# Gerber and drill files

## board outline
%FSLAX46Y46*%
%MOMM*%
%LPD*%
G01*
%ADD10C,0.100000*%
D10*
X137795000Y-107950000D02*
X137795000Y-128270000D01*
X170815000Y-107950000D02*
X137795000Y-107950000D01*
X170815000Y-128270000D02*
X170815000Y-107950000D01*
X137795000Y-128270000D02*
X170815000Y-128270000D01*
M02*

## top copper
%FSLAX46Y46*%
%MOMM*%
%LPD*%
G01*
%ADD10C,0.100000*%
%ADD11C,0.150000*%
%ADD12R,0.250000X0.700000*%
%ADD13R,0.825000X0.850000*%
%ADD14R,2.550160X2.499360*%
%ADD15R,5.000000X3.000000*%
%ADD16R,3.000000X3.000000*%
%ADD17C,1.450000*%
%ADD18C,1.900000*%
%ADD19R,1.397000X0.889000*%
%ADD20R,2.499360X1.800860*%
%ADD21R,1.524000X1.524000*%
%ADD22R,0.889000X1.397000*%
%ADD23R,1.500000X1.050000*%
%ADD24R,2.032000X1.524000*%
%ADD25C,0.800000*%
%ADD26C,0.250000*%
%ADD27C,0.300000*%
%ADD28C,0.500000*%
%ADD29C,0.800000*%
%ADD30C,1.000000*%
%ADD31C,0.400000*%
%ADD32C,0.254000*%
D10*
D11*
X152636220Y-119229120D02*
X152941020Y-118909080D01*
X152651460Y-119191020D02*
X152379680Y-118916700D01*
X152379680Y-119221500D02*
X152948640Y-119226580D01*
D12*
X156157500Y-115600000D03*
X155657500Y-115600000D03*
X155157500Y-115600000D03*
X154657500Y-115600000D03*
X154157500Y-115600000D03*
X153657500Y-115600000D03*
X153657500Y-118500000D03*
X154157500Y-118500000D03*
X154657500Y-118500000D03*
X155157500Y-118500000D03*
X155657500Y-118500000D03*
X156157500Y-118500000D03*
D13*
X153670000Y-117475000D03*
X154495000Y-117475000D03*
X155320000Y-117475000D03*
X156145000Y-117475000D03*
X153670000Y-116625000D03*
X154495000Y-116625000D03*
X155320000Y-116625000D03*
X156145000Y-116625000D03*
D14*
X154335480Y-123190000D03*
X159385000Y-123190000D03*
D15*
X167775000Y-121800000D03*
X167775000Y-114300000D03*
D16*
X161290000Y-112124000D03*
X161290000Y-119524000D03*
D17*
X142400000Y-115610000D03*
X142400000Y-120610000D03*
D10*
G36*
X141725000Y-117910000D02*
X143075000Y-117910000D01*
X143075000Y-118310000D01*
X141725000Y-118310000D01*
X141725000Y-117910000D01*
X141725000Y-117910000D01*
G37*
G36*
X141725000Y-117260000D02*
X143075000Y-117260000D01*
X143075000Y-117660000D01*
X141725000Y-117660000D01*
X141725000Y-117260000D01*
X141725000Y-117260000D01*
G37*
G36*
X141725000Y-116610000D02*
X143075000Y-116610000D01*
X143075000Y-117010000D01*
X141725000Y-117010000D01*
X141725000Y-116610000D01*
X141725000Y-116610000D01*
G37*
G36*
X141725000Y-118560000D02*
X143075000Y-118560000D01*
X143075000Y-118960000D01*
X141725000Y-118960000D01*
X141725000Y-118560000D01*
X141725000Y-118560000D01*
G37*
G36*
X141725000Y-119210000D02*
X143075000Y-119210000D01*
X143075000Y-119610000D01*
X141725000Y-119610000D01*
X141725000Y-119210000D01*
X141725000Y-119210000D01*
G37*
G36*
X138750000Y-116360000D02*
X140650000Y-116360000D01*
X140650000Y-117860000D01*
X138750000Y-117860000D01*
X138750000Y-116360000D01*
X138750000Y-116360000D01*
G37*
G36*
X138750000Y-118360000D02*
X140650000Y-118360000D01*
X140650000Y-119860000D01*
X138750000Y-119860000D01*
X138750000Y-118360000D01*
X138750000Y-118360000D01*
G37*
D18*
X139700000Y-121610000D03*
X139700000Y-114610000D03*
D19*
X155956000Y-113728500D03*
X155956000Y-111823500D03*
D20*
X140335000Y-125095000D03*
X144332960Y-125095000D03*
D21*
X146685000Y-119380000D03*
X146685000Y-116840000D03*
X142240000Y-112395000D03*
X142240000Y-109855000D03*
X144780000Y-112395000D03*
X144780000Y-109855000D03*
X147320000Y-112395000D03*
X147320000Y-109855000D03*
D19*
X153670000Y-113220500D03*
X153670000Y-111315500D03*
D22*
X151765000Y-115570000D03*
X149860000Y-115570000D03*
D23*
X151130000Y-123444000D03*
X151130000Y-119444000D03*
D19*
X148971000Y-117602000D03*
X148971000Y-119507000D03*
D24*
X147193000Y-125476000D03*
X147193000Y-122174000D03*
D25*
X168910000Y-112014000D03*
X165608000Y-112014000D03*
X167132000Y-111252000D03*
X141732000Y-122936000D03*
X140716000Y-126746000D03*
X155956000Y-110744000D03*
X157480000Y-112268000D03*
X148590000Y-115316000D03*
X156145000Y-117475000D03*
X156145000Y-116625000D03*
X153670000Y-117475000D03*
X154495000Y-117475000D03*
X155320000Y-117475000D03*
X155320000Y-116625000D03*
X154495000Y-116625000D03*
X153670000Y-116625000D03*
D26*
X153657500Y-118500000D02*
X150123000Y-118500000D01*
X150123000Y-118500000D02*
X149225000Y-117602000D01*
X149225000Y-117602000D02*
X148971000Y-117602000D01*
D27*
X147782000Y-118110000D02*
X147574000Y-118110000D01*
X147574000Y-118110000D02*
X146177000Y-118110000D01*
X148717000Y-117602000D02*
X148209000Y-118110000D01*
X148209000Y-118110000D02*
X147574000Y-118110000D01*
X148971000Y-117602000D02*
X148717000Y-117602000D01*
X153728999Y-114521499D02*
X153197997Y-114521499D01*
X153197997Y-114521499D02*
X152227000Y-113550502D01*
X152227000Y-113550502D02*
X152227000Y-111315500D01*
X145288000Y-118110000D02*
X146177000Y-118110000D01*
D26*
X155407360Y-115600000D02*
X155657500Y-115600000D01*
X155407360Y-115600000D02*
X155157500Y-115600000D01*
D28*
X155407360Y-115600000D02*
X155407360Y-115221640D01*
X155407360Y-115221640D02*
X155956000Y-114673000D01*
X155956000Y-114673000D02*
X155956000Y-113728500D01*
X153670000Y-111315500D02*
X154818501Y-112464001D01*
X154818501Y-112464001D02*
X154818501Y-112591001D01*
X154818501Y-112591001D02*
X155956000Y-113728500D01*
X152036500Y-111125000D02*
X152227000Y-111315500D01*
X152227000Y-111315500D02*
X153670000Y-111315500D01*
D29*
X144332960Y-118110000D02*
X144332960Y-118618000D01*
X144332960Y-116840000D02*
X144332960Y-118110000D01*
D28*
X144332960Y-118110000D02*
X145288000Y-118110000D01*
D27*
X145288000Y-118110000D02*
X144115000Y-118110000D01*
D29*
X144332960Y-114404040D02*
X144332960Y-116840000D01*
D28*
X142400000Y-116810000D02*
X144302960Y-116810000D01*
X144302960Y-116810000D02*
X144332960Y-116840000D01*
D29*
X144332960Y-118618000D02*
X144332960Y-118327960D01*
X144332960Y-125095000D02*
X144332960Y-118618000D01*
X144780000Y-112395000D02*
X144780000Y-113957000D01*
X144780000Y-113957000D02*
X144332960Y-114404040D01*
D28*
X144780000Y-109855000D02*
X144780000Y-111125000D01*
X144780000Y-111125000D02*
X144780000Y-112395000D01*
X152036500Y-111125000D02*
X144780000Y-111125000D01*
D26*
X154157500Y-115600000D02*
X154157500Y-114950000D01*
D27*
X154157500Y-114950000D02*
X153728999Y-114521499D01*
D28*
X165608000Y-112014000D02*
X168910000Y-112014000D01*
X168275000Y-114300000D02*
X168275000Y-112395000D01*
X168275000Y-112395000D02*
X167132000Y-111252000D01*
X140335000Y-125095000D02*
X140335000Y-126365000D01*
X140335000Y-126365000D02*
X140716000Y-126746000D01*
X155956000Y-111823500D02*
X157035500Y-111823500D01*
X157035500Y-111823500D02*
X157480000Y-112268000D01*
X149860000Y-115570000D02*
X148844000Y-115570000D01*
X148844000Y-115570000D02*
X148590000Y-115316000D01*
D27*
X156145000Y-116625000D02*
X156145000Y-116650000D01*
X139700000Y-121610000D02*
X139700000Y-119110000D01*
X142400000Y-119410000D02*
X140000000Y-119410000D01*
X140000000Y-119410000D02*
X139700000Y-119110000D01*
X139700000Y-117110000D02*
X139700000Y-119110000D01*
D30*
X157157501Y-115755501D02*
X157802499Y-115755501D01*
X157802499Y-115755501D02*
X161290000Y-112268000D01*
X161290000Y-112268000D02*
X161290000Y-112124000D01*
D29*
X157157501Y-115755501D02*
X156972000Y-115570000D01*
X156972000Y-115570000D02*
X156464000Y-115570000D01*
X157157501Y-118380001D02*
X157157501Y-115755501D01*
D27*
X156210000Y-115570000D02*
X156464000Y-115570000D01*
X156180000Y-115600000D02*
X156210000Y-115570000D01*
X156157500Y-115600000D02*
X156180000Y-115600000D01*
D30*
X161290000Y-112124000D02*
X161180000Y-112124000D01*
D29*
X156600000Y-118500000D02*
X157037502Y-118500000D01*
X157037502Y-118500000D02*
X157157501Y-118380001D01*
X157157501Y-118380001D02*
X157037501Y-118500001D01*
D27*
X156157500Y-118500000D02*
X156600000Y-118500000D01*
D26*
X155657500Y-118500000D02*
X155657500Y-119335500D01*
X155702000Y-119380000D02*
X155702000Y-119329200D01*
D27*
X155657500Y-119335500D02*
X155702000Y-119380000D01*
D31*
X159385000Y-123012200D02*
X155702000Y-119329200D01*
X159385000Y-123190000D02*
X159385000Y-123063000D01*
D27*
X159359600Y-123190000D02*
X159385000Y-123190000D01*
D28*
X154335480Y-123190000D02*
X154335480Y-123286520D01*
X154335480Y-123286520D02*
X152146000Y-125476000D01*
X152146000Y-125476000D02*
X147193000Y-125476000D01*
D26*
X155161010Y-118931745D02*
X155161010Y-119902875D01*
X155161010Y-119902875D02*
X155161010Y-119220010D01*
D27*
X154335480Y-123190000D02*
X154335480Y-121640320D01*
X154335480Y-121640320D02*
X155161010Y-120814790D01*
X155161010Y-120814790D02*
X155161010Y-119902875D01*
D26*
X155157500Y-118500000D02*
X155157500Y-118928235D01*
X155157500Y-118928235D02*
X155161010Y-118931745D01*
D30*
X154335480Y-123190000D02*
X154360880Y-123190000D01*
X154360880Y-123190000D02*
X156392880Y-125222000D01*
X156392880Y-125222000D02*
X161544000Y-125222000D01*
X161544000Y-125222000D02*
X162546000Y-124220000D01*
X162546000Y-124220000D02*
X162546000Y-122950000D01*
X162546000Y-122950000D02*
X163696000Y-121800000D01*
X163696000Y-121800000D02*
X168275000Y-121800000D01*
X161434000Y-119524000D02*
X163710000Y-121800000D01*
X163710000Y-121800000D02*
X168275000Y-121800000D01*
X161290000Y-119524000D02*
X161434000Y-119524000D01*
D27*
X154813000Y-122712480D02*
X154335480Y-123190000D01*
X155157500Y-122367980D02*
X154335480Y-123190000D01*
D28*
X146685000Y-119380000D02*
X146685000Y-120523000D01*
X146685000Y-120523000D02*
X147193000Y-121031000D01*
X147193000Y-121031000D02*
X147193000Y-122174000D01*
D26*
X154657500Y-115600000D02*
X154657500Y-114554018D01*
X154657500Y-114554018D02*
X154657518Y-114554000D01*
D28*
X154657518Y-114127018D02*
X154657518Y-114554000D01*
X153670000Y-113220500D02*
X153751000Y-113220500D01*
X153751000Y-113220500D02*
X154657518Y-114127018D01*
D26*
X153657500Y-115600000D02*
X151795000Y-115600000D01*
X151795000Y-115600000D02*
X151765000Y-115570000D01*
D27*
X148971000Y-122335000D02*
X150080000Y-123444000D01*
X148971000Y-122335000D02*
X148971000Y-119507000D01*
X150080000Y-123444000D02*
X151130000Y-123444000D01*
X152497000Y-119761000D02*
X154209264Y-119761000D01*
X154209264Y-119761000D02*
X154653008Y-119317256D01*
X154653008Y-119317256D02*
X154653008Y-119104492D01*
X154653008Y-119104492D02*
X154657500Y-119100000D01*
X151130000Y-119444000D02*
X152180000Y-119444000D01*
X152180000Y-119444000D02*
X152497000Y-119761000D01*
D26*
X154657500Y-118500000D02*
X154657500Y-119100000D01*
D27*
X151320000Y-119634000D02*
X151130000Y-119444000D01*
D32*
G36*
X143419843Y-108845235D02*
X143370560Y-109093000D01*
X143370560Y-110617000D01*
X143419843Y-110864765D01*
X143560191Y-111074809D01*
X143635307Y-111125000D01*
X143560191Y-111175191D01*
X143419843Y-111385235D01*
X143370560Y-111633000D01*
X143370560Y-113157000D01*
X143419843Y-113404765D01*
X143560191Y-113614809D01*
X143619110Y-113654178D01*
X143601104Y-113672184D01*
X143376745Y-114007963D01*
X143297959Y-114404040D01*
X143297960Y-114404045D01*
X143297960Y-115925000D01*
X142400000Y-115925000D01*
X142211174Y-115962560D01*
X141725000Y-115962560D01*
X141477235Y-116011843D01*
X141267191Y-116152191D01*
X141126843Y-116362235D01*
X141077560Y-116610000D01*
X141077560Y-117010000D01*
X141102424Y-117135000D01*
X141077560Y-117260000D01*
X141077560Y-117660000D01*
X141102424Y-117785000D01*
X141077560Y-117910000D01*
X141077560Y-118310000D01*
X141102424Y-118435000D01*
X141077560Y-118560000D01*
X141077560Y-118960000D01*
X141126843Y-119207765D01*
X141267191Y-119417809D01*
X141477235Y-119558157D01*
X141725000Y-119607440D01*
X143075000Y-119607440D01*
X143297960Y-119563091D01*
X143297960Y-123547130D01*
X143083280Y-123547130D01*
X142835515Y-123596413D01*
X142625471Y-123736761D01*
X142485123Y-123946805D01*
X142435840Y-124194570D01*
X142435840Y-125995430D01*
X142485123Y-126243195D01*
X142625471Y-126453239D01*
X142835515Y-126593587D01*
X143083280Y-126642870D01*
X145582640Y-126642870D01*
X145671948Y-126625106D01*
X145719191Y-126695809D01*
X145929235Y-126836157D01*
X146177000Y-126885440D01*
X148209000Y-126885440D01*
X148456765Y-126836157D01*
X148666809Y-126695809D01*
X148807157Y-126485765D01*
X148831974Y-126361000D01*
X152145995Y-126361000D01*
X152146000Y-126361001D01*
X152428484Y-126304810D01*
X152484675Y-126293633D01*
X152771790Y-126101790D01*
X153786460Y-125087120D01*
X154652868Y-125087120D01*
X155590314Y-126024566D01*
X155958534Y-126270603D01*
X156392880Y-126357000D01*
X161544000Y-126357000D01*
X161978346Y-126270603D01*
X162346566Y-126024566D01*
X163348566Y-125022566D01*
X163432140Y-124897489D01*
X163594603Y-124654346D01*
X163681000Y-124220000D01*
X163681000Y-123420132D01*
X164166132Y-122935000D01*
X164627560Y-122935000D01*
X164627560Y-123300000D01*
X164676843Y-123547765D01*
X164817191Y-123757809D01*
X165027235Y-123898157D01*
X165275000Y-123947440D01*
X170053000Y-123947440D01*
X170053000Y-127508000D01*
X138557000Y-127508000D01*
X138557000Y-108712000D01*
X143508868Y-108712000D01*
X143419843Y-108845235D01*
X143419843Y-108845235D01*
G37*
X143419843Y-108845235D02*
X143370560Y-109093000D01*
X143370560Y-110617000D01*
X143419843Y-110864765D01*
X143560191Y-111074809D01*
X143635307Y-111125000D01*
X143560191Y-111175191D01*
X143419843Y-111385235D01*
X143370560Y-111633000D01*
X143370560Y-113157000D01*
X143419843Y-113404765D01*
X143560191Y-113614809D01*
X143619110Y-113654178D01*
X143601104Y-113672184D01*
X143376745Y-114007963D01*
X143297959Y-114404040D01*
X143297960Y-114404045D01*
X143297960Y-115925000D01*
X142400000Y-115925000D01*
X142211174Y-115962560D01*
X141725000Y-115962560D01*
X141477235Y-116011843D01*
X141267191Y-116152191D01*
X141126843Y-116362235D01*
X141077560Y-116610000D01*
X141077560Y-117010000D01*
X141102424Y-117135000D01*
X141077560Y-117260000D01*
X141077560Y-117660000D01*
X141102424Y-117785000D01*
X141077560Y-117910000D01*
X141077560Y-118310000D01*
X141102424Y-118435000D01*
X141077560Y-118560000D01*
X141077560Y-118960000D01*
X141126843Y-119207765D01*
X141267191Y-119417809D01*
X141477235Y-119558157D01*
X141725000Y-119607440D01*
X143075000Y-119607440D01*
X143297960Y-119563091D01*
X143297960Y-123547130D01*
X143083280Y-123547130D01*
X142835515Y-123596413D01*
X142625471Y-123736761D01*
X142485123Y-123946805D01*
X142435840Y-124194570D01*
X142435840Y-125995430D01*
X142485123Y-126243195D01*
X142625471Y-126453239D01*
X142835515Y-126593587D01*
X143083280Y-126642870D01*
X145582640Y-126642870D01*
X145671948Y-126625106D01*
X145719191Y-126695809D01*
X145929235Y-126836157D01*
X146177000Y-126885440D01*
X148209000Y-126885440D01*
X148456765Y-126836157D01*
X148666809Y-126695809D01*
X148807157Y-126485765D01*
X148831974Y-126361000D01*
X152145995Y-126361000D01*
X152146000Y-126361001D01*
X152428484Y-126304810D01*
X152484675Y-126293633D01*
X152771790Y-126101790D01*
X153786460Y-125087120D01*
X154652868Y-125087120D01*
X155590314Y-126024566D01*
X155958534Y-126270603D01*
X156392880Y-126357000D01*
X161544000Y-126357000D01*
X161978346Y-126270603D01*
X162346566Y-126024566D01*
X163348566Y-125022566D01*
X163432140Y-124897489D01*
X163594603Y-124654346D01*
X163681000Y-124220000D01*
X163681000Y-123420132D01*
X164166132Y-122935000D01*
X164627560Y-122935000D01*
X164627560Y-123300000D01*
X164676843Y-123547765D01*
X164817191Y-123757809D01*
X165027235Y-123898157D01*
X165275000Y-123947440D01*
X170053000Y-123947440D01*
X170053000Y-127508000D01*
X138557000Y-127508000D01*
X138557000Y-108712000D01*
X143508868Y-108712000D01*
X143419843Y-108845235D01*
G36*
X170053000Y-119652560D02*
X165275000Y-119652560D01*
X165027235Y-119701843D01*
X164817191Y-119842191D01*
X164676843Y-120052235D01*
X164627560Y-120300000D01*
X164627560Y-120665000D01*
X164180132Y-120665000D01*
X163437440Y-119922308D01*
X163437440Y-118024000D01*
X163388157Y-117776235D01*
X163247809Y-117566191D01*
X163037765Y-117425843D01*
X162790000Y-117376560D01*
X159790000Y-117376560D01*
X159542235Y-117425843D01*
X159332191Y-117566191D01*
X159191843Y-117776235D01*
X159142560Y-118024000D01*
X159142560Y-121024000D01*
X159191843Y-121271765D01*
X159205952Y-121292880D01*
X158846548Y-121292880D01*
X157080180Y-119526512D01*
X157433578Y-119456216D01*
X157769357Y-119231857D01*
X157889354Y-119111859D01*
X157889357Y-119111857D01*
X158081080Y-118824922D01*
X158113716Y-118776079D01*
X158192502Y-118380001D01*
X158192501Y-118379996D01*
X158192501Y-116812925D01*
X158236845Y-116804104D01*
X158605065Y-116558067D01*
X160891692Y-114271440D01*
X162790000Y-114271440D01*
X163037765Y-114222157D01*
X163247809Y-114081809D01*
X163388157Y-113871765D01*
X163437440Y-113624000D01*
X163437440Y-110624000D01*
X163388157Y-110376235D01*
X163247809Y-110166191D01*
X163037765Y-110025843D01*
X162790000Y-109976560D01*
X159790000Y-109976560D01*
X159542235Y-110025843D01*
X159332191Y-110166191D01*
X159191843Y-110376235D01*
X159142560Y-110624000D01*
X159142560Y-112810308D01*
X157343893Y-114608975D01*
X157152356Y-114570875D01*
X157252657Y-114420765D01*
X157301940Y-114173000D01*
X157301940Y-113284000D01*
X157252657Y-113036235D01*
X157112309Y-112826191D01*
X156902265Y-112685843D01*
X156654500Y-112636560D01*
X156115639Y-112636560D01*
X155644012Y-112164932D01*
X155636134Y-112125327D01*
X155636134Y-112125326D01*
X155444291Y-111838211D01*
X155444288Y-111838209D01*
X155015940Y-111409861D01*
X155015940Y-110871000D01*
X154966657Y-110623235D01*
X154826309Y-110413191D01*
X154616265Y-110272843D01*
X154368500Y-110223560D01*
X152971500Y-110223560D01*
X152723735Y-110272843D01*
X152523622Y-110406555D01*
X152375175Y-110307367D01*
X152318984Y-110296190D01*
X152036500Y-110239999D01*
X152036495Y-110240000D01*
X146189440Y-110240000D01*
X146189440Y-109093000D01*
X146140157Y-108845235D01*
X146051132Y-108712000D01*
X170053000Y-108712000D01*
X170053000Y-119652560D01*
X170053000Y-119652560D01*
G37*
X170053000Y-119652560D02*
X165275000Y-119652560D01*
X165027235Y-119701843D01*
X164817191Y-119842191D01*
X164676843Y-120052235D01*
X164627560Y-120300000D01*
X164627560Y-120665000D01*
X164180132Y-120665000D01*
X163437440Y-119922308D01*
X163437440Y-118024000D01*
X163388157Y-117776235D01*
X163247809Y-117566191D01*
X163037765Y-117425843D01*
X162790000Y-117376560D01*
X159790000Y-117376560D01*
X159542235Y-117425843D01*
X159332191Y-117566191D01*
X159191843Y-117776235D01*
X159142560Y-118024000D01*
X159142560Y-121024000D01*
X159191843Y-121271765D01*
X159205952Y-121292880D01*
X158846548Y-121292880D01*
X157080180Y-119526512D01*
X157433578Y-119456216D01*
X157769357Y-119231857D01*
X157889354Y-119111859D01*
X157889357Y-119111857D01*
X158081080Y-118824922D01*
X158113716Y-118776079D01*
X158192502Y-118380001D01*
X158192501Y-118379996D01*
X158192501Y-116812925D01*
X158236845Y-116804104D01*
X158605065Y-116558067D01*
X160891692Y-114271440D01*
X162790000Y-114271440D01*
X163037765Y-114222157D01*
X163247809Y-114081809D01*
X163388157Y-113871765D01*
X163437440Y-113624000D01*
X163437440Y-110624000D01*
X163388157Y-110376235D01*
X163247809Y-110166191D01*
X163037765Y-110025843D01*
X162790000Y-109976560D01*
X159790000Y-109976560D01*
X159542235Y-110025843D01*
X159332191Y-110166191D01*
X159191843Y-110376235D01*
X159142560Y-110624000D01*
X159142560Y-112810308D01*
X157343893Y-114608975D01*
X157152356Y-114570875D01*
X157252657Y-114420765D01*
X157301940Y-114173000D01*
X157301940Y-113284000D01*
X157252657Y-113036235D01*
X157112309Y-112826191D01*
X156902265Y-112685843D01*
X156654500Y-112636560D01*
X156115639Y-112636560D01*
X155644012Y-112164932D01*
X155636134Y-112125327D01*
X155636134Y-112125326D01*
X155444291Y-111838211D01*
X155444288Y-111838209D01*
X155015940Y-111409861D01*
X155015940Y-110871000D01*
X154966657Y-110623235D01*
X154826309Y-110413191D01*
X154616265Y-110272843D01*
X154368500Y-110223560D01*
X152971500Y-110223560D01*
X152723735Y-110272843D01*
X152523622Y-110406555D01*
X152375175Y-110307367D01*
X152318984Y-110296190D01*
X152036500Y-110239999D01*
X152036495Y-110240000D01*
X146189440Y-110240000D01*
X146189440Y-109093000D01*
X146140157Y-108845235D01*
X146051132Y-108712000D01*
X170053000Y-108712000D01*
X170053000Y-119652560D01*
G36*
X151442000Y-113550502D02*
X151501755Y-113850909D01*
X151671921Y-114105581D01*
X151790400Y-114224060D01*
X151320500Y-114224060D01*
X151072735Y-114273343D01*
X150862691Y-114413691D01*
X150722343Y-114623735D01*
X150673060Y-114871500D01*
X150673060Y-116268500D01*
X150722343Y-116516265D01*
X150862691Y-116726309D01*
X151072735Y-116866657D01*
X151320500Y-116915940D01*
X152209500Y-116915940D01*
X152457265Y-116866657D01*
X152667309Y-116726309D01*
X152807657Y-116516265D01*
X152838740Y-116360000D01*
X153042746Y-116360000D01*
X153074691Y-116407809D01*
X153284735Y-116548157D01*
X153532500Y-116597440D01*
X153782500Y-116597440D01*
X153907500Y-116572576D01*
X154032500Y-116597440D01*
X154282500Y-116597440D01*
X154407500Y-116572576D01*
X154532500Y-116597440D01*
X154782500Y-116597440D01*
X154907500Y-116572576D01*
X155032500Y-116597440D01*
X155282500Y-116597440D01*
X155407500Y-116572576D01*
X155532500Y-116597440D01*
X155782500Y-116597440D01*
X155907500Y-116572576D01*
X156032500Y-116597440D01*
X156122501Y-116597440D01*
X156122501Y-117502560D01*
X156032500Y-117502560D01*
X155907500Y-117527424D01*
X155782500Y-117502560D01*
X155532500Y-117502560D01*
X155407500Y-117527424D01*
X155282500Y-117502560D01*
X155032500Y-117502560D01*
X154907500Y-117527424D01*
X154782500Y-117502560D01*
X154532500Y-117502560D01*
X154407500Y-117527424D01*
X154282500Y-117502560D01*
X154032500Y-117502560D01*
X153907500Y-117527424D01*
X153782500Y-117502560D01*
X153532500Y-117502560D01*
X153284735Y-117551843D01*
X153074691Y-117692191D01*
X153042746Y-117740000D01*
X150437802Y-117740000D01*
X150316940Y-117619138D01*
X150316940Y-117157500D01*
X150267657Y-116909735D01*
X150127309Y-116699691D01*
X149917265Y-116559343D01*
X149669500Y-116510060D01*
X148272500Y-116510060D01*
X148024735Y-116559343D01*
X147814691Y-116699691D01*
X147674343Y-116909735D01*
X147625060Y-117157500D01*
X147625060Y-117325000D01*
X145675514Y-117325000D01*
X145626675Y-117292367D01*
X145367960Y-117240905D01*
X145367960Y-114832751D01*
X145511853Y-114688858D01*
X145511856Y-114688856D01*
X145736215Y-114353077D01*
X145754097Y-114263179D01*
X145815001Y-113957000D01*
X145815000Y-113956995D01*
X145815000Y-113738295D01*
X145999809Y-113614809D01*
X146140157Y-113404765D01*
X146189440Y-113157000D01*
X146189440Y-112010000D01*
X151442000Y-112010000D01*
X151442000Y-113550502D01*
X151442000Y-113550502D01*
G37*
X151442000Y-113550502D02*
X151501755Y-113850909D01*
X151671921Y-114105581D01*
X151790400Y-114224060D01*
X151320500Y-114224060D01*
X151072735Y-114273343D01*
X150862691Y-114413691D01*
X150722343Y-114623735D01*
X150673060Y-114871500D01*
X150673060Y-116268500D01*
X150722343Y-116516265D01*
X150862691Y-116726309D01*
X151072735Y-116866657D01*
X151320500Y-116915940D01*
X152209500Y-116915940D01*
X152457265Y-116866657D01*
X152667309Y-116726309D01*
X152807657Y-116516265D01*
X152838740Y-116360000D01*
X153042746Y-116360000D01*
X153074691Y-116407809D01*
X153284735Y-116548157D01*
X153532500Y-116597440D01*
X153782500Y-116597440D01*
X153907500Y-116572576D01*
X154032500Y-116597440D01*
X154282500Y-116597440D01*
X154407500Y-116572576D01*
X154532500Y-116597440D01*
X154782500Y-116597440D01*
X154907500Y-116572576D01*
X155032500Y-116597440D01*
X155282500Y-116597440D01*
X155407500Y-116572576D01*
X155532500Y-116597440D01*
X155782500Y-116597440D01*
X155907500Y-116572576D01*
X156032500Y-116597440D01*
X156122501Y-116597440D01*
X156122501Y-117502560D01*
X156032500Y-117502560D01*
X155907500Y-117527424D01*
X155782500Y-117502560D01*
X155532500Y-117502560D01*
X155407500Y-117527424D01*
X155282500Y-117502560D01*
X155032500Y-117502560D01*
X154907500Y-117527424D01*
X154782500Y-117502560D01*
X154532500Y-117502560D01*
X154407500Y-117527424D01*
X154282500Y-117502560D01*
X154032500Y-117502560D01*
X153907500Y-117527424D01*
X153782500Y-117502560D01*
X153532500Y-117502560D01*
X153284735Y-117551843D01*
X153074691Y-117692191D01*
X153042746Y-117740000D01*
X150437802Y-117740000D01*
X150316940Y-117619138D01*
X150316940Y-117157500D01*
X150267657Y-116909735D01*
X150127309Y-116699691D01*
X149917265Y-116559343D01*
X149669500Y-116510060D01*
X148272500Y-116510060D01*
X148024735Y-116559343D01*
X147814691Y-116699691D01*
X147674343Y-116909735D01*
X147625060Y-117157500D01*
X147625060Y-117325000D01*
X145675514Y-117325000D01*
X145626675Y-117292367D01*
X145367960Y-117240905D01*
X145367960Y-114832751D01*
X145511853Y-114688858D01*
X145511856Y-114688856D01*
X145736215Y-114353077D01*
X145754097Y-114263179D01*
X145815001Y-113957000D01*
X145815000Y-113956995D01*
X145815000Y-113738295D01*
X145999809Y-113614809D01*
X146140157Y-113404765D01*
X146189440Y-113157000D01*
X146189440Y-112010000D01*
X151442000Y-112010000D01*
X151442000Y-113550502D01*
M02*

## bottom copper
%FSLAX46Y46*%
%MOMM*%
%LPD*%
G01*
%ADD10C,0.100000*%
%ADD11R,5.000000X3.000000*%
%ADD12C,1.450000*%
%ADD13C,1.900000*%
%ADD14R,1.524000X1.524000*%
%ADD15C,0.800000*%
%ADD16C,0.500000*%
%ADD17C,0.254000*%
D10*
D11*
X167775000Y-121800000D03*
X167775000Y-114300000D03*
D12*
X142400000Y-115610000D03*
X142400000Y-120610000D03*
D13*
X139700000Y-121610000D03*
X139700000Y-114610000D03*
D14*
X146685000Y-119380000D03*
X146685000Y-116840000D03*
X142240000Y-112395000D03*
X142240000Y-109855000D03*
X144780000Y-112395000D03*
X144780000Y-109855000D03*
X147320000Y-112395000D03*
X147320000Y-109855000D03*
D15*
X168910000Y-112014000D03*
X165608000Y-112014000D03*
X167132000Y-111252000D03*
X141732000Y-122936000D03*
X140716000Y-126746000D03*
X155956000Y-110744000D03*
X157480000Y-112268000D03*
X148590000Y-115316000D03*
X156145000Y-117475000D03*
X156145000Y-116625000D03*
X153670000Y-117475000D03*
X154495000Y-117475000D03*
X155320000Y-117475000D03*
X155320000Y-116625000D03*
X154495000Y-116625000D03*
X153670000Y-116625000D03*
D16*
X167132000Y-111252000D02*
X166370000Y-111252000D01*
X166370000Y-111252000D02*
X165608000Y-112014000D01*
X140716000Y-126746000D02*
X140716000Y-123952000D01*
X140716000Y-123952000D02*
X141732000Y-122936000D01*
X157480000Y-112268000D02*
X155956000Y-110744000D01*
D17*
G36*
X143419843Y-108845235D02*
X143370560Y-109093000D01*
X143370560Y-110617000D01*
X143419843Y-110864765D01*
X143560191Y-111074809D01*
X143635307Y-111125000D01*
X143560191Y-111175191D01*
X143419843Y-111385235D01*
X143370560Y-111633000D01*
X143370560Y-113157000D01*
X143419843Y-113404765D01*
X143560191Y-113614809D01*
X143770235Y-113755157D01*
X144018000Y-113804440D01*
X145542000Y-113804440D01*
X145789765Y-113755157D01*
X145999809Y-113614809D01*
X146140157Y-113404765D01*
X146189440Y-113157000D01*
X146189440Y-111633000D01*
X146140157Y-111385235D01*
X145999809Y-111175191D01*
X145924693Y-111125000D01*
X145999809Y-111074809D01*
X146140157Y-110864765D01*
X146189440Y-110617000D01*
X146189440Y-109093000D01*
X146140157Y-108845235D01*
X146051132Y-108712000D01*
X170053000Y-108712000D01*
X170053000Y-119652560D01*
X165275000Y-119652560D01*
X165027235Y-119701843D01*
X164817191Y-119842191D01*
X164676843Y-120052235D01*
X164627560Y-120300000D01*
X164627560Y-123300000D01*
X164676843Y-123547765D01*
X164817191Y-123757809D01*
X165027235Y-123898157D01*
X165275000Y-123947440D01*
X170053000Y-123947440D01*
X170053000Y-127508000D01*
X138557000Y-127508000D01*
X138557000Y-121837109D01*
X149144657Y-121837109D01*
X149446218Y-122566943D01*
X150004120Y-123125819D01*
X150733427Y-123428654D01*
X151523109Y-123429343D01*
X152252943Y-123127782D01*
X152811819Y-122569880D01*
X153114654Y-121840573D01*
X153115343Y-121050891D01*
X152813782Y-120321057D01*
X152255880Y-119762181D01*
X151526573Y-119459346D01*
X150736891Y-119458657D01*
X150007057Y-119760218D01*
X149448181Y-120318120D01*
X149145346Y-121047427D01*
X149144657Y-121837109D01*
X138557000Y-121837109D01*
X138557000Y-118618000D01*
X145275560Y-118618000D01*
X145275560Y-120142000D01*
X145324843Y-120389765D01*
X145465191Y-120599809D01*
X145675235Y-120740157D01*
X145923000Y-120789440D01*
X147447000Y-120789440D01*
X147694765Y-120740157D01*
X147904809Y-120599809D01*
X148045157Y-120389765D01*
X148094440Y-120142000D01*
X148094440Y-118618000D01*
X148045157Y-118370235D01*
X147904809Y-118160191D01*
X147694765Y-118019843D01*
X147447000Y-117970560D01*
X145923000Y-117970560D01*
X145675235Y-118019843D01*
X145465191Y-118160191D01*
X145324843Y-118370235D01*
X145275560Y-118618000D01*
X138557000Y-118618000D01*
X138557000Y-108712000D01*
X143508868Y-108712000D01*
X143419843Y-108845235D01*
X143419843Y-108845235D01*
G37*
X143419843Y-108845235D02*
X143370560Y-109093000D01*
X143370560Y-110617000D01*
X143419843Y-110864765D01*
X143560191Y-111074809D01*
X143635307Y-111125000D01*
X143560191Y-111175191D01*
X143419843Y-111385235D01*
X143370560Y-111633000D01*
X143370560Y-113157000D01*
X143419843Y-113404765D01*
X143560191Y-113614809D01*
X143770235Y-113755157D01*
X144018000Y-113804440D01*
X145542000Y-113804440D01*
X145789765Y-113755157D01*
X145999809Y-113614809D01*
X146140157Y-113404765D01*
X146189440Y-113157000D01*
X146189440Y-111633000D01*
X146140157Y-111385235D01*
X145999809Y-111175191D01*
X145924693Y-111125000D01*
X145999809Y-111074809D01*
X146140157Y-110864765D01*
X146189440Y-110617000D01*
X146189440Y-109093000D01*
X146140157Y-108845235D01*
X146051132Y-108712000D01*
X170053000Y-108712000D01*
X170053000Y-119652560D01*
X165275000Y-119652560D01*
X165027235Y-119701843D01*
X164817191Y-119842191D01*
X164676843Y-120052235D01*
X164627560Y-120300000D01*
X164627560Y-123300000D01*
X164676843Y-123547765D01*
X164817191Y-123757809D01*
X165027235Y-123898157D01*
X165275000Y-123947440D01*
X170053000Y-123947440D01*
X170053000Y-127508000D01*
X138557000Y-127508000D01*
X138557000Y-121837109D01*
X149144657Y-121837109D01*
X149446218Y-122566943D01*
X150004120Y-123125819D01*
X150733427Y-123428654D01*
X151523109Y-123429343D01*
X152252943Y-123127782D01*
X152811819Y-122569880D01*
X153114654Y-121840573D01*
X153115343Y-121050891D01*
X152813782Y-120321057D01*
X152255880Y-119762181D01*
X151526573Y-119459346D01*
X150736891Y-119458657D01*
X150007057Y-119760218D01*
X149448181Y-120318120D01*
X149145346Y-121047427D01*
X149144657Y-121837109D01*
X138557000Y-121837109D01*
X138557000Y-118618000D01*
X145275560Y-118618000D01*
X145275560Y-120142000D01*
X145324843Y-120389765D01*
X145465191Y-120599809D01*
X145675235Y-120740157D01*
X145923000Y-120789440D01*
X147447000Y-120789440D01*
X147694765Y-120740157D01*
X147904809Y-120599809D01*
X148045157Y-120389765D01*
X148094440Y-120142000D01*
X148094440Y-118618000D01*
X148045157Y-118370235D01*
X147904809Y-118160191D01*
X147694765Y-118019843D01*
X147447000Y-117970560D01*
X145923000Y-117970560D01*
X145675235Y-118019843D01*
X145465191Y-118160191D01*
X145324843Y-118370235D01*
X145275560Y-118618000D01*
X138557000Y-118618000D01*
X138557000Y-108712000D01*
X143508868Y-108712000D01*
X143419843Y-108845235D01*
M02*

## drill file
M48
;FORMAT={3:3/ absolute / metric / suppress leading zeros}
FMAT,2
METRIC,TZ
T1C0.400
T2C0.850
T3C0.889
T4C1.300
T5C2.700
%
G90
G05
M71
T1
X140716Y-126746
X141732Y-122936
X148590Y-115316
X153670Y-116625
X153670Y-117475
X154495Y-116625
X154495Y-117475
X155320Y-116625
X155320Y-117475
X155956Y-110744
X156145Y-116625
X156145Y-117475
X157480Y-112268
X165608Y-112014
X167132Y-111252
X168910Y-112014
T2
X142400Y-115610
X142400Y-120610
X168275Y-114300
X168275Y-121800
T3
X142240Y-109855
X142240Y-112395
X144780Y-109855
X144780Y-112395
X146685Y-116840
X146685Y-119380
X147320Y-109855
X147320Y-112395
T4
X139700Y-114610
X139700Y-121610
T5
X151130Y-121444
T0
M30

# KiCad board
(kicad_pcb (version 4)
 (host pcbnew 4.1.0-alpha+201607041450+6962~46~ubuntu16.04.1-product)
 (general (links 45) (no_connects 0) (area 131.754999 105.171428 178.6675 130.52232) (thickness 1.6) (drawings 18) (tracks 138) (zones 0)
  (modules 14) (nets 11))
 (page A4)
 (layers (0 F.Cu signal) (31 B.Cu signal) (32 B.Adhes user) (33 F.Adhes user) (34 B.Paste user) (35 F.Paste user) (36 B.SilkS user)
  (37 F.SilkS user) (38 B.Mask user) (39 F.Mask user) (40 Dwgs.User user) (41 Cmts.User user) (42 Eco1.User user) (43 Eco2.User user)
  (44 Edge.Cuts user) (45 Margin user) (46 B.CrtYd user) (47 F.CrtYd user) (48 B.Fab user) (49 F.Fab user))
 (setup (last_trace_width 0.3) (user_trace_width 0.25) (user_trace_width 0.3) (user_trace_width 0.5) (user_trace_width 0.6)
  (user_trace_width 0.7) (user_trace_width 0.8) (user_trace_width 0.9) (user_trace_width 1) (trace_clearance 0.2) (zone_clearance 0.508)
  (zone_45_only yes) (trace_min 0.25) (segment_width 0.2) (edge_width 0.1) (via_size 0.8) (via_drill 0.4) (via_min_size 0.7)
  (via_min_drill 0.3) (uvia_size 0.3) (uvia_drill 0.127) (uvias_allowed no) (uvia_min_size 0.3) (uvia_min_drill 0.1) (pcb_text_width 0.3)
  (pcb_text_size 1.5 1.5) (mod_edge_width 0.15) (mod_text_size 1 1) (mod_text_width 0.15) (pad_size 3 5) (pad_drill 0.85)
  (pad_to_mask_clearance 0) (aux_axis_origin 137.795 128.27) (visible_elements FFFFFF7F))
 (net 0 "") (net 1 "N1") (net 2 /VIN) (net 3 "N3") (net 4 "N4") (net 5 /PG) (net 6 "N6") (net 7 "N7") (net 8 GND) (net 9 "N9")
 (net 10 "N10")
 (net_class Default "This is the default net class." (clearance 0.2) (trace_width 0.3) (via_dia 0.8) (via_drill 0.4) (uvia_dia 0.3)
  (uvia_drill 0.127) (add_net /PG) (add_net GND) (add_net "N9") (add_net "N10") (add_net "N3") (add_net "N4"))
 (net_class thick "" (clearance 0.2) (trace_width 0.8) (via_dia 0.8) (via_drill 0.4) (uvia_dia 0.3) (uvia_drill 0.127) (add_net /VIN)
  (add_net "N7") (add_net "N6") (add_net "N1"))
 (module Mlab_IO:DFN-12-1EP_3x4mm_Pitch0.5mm (layer F.Cu) (at 154.9075 117.05 270)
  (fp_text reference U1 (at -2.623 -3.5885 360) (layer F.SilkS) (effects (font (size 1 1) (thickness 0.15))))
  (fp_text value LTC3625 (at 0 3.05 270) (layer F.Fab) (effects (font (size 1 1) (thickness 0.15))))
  (pad 1 smd rect (at -1.45 -1.25 270) (size 0.7 0.25) (layers F.Cu F.Paste F.Mask) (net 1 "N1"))
  (pad 2 smd rect (at -1.45 -0.75 270) (size 0.7 0.25) (layers F.Cu F.Paste F.Mask) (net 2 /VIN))
  (pad 3 smd rect (at -1.45 -0.25 270) (size 0.7 0.25) (layers F.Cu F.Paste F.Mask) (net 2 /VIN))
  (pad 4 smd rect (at -1.45 0.25 270) (size 0.7 0.25) (layers F.Cu F.Paste F.Mask) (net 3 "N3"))
  (pad 5 smd rect (at -1.45 0.75 270) (size 0.7 0.25) (layers F.Cu F.Paste F.Mask) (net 2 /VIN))
  (pad 6 smd rect (at -1.45 1.25 270) (size 0.7 0.25) (layers F.Cu F.Paste F.Mask) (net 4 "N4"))
  (pad 7 smd rect (at 1.45 1.25 270) (size 0.7 0.25) (layers F.Cu F.Paste F.Mask) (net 2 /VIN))
  (pad 8 smd rect (at 1.45 0.75 270) (size 0.7 0.25) (layers F.Cu F.Paste F.Mask))
  (pad 9 smd rect (at 1.45 0.25 270) (size 0.7 0.25) (layers F.Cu F.Paste F.Mask) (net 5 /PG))
  (pad 10 smd rect (at 1.45 -0.25 270) (size 0.7 0.25) (layers F.Cu F.Paste F.Mask) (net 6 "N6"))
  (pad 11 smd rect (at 1.45 -0.75 270) (size 0.7 0.25) (layers F.Cu F.Paste F.Mask) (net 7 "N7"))
  (pad 12 smd rect (at 1.45 -1.25 270) (size 0.7 0.25) (layers F.Cu F.Paste F.Mask) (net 1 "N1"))
  (pad 13 smd rect (at 0.425 1.2375 270) (size 0.85 0.825) (layers F.Cu F.Paste F.Mask) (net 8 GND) (solder_paste_margin_ratio -0.2))
  (pad 13 smd rect (at 0.425 0.4125 270) (size 0.85 0.825) (layers F.Cu F.Paste F.Mask) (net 8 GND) (solder_paste_margin_ratio -0.2))
  (pad 13 smd rect (at 0.425 -0.4125 270) (size 0.85 0.825) (layers F.Cu F.Paste F.Mask) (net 8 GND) (solder_paste_margin_ratio -0.2))
  (pad 13 smd rect (at 0.425 -1.2375 270) (size 0.85 0.825) (layers F.Cu F.Paste F.Mask) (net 8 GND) (solder_paste_margin_ratio -0.2))
  (pad 13 smd rect (at -0.425 1.2375 270) (size 0.85 0.825) (layers F.Cu F.Paste F.Mask) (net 8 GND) (solder_paste_margin_ratio -0.2))
  (pad 13 smd rect (at -0.425 0.4125 270) (size 0.85 0.825) (layers F.Cu F.Paste F.Mask) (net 8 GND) (solder_paste_margin_ratio -0.2))
  (pad 13 smd rect (at -0.425 -0.4125 270) (size 0.85 0.825) (layers F.Cu F.Paste F.Mask) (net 8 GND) (solder_paste_margin_ratio -0.2))
  (pad 13 smd rect (at -0.425 -1.2375 270) (size 0.85 0.825) (layers F.Cu F.Paste F.Mask) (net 8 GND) (solder_paste_margin_ratio -0.2)))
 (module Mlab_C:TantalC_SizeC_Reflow (layer F.Cu) (at 156.86024 123.19 180)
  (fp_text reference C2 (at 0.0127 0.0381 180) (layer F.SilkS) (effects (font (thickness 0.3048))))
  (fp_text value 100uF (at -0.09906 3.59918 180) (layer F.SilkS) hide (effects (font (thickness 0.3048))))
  (pad 2 smd rect (at 2.52476 0 180) (size 2.55016 2.49936) (layers F.Cu F.Paste F.Mask) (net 6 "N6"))
  (pad 1 smd rect (at -2.52476 0 180) (size 2.55016 2.49936) (layers F.Cu F.Paste F.Mask) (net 7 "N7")))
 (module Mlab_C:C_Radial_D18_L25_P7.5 (layer B.Cu) (at 168.275 121.8 90)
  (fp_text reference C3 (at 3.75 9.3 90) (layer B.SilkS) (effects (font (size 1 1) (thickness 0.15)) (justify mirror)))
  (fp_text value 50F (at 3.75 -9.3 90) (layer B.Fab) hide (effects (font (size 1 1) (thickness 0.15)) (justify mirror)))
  (pad 1 thru_hole rect (at 0 0 90) (size 3 5) (drill 0.85 (offset 0 -0.5)) (layers *.Cu *.Mask B.SilkS) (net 6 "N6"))
  (pad 2 thru_hole rect (at 7.5 0 90) (size 3 5) (drill 0.85 (offset 0 -0.5)) (layers *.Cu *.Mask B.SilkS) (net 8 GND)))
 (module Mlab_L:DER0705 (layer F.Cu) (at 161.29 115.824 90)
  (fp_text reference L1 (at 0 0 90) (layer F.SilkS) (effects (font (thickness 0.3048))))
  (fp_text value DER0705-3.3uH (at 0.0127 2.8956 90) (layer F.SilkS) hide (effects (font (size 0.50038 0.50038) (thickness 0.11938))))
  (pad 1 smd rect (at 3.7 0 90) (size 3 3) (layers F.Cu F.Paste F.Mask) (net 1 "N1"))
  (pad 2 smd rect (at -3.7 0 90) (size 3 3) (layers F.Cu F.Paste F.Mask) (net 6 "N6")))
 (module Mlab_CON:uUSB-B (layer F.Cu) (at 139.7 118.11 270)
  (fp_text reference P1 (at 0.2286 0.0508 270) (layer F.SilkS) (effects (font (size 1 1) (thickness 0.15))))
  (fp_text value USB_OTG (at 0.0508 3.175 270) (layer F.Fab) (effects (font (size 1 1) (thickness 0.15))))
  (pad 5 thru_hole circle (at -2.5 -2.7 270) (size 1.45 1.45) (drill 0.85) (layers *.Cu *.Mask) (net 8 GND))
  (pad 5 thru_hole circle (at 2.5 -2.7 270) (size 1.45 1.45) (drill 0.85) (layers *.Cu *.Mask) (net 8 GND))
  (pad 3 smd trapezoid (at 0 -2.7 270) (size 0.4 1.35) (layers F.Cu F.Mask))
  (pad 2 smd trapezoid (at -0.65 -2.7 270) (size 0.4 1.35) (layers F.Cu F.Mask))
  (pad 1 smd trapezoid (at -1.3 -2.7 270) (size 0.4 1.35) (layers F.Cu F.Mask) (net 2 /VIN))
  (pad 4 smd trapezoid (at 0.65 -2.7 270) (size 0.4 1.35) (layers F.Cu F.Mask))
  (pad 5 smd trapezoid (at 1.3 -2.7 270) (size 0.4 1.35) (layers F.Cu F.Mask) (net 8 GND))
  (pad 5 smd trapezoid (at -1 0 270) (size 1.5 1.9) (layers F.Cu F.Mask) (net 8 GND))
  (pad 5 smd trapezoid (at 1 0 270) (size 1.5 1.9) (layers F.Cu F.Mask) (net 8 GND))
  (pad 5 thru_hole circle (at 3.5 0 270) (size 1.9 1.9) (drill 1.3) (layers *.Cu *.Mask) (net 8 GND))
  (pad 5 thru_hole circle (at -3.5 0 270) (size 1.9 1.9) (drill 1.3) (layers *.Cu *.Mask) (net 8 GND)))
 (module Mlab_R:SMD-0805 (layer F.Cu) (at 155.956 112.776 90)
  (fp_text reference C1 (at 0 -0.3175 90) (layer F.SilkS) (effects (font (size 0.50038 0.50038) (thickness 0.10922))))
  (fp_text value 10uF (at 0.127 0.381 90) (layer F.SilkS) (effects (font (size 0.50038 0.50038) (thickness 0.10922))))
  (pad 1 smd rect (at -0.9525 0 90) (size 0.889 1.397) (layers F.Cu F.Paste F.Mask) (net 2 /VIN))
  (pad 2 smd rect (at 0.9525 0 90) (size 0.889 1.397) (layers F.Cu F.Paste F.Mask) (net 8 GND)))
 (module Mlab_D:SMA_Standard (layer F.Cu) (at 142.33398 125.095)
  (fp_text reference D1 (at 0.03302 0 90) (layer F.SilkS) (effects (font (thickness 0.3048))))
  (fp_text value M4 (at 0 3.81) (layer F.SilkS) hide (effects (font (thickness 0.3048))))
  (pad 1 smd rect (at -1.99898 0) (size 2.49936 1.80086) (layers F.Cu F.Paste F.Mask) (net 8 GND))
  (pad 2 smd rect (at 1.99898 0) (size 2.49936 1.80086) (layers F.Cu F.Paste F.Mask) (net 2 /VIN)))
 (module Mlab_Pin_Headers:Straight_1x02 (layer F.Cu) (at 146.685 118.11)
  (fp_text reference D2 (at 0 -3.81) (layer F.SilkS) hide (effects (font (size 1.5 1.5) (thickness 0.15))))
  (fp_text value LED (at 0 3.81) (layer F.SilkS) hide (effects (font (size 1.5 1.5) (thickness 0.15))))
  (pad 2 thru_hole rect (at 0 1.27) (size 1.524 1.524) (drill 0.889) (layers *.Cu *.Mask F.SilkS) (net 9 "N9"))
  (pad 1 thru_hole rect (at 0 -1.27) (size 1.524 1.524) (drill 0.889) (layers *.Cu *.Mask F.SilkS) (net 8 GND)))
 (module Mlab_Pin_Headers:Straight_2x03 (layer F.Cu) (at 144.78 111.125 90)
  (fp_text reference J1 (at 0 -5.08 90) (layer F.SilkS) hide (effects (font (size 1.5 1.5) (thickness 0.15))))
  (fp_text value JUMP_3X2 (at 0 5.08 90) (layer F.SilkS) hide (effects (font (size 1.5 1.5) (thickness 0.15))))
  (pad 1 thru_hole rect (at -1.27 -2.54 90) (size 1.524 1.524) (drill 0.889) (layers *.Cu *.Mask F.SilkS) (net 8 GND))
  (pad 2 thru_hole rect (at 1.27 -2.54 90) (size 1.524 1.524) (drill 0.889) (layers *.Cu *.Mask F.SilkS) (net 8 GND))
  (pad 3 thru_hole rect (at -1.27 0 90) (size 1.524 1.524) (drill 0.889) (layers *.Cu *.Mask F.SilkS) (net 2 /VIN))
  (pad 4 thru_hole rect (at 1.27 0 90) (size 1.524 1.524) (drill 0.889) (layers *.Cu *.Mask F.SilkS) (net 2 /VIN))
  (pad 5 thru_hole rect (at -1.27 2.54 90) (size 1.524 1.524) (drill 0.889) (layers *.Cu *.Mask F.SilkS) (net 8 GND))
  (pad 6 thru_hole rect (at 1.27 2.54 90) (size 1.524 1.524) (drill 0.889) (layers *.Cu *.Mask F.SilkS) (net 8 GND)))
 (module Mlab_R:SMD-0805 (layer F.Cu) (at 153.67 112.268 90)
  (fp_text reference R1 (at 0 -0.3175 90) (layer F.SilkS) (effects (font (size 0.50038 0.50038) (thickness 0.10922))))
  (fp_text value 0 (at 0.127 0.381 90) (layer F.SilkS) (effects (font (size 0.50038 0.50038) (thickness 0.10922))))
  (pad 1 smd rect (at -0.9525 0 90) (size 0.889 1.397) (layers F.Cu F.Paste F.Mask) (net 3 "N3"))
  (pad 2 smd rect (at 0.9525 0 90) (size 0.889 1.397) (layers F.Cu F.Paste F.Mask) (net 2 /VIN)))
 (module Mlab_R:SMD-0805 (layer F.Cu) (at 150.8125 115.57 180)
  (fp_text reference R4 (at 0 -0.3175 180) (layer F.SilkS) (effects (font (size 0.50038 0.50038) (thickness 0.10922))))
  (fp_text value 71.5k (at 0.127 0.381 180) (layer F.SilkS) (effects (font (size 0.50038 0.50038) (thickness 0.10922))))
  (pad 1 smd rect (at -0.9525 0 180) (size 0.889 1.397) (layers F.Cu F.Paste F.Mask) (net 4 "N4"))
  (pad 2 smd rect (at 0.9525 0 180) (size 0.889 1.397) (layers F.Cu F.Paste F.Mask) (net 8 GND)))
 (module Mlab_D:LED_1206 (layer F.Cu) (at 151.13 121.444 90)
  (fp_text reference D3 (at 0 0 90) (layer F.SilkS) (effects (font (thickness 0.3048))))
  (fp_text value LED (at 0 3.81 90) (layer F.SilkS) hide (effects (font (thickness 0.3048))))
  (fp_line (start 2.21488 1.50622) (end 2.53492 1.81102) (layer F.Cu) (width 0.15))
  (fp_line (start 2.25298 1.52146) (end 2.5273 1.24968) (layer F.Cu) (width 0.15))
  (fp_line (start 2.2225 1.24968) (end 2.21742 1.81864) (layer F.Cu) (width 0.15))
  (pad 2 smd rect (at -2 0 90) (size 1.05 1.5) (layers F.Cu F.Paste F.Mask) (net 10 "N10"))
  (pad 1 smd rect (at 2 0 90) (size 1.05 1.5) (layers F.Cu F.Paste F.Mask) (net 5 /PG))
  (pad "" np_thru_hole circle (at 0 0 90) (size 2.7 2.7) (drill 2.7) (layers *.Cu *.Mask F.SilkS)))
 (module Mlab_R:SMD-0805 (layer F.Cu) (at 148.971 118.5545 270)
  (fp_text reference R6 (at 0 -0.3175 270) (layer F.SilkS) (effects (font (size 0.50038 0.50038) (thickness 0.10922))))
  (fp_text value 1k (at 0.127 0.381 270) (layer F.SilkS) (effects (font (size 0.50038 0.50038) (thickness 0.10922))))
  (pad 1 smd rect (at -0.9525 0 270) (size 0.889 1.397) (layers F.Cu F.Paste F.Mask) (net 2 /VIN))
  (pad 2 smd rect (at 0.9525 0 270) (size 0.889 1.397) (layers F.Cu F.Paste F.Mask) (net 10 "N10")))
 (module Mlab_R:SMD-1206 (layer F.Cu) (at 147.193 123.825 90)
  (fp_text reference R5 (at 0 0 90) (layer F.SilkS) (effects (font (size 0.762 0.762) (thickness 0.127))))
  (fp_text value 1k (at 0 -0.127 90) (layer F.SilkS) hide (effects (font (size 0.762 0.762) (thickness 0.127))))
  (pad 1 smd rect (at -1.651 0 90) (size 1.524 2.032) (layers F.Cu F.Paste F.Mask) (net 6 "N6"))
  (pad 2 smd rect (at 1.651 0 90) (size 1.524 2.032) (layers F.Cu F.Paste F.Mask) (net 9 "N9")))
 (gr_line (start 137.795 107.95) (end 137.795 128.27) (angle 90) (layer Edge.Cuts) (width 0.1))
 (gr_line (start 170.815 107.95) (end 137.795 107.95) (angle 90) (layer Edge.Cuts) (width 0.1))
 (gr_line (start 170.815 128.27) (end 170.815 107.95) (angle 90) (layer Edge.Cuts) (width 0.1))
 (gr_line (start 137.795 128.27) (end 170.815 128.27) (angle 90) (layer Edge.Cuts) (width 0.1))
 (segment (start 176.53 130.175) (end 176.53 120.65) (width 0.25) (layer Dwgs.User) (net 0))
 (segment (start 132.08 113.03) (end 134.62 110.49) (width 0.25) (layer Dwgs.User) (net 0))
 (segment (start 153.6575 118.5) (end 150.123 118.5) (width 0.25) (layer F.Cu) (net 2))
 (segment (start 150.123 118.5) (end 149.225 117.602) (width 0.25) (layer F.Cu) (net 2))
 (segment (start 149.225 117.602) (end 148.971 117.602) (width 0.25) (layer F.Cu) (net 2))
 (segment (start 147.782 118.11) (end 147.574 118.11) (width 0.3) (layer F.Cu) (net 2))
 (segment (start 147.574 118.11) (end 146.177 118.11) (width 0.3) (layer F.Cu) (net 2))
 (segment (start 148.717 117.602) (end 148.209 118.11) (width 0.3) (layer F.Cu) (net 2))
 (segment (start 148.209 118.11) (end 147.574 118.11) (width 0.3) (layer F.Cu) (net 2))
 (segment (start 148.971 117.602) (end 148.717 117.602) (width 0.3) (layer F.Cu) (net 2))
 (segment (start 153.728999 114.521499) (end 153.197997 114.521499) (width 0.3) (layer F.Cu) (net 2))
 (segment (start 153.197997 114.521499) (end 152.227 113.550502) (width 0.3) (layer F.Cu) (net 2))
 (segment (start 152.227 113.550502) (end 152.227 111.3155) (width 0.3) (layer F.Cu) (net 2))
 (segment (start 145.288 118.11) (end 146.177 118.11) (width 0.3) (layer F.Cu) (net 2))
 (segment (start 155.40736 115.6) (end 155.6575 115.6) (width 0.25) (layer F.Cu) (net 2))
 (segment (start 155.40736 115.6) (end 155.1575 115.6) (width 0.25) (layer F.Cu) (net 2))
 (segment (start 155.40736 115.6) (end 155.40736 115.22164) (width 0.5) (layer F.Cu) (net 2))
 (segment (start 155.40736 115.22164) (end 155.956 114.673) (width 0.5) (layer F.Cu) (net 2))
 (segment (start 155.956 114.673) (end 155.956 113.7285) (width 0.5) (layer F.Cu) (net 2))
 (segment (start 153.67 111.3155) (end 154.818501 112.464001) (width 0.5) (layer F.Cu) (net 2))
 (segment (start 154.818501 112.464001) (end 154.818501 112.591001) (width 0.5) (layer F.Cu) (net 2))
 (segment (start 154.818501 112.591001) (end 155.956 113.7285) (width 0.5) (layer F.Cu) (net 2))
 (segment (start 152.0365 111.125) (end 152.227 111.3155) (width 0.5) (layer F.Cu) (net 2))
 (segment (start 152.227 111.3155) (end 153.67 111.3155) (width 0.5) (layer F.Cu) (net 2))
 (segment (start 144.33296 118.11) (end 144.33296 118.618) (width 0.8) (layer F.Cu) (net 2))
 (segment (start 144.33296 116.84) (end 144.33296 118.11) (width 0.8) (layer F.Cu) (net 2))
 (segment (start 144.33296 118.11) (end 145.288 118.11) (width 0.5) (layer F.Cu) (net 2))
 (segment (start 145.288 118.11) (end 144.115 118.11) (width 0.3) (layer F.Cu) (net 2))
 (segment (start 144.33296 114.40404) (end 144.33296 116.84) (width 0.8) (layer F.Cu) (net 2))
 (segment (start 142.4 116.81) (end 144.30296 116.81) (width 0.5) (layer F.Cu) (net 2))
 (segment (start 144.30296 116.81) (end 144.33296 116.84) (width 0.5) (layer F.Cu) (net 2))
 (segment (start 144.33296 118.618) (end 144.33296 118.32796) (width 0.8) (layer F.Cu) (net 2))
 (segment (start 144.33296 125.095) (end 144.33296 118.618) (width 0.8) (layer F.Cu) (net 2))
 (segment (start 144.78 112.395) (end 144.78 113.957) (width 0.8) (layer F.Cu) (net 2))
 (segment (start 144.78 113.957) (end 144.33296 114.40404) (width 0.8) (layer F.Cu) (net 2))
 (segment (start 144.78 109.855) (end 144.78 111.125) (width 0.5) (layer F.Cu) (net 2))
 (segment (start 144.78 111.125) (end 144.78 112.395) (width 0.5) (layer F.Cu) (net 2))
 (segment (start 152.0365 111.125) (end 144.78 111.125) (width 0.5) (layer F.Cu) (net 2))
 (segment (start 154.1575 115.6) (end 154.1575 114.95) (width 0.25) (layer F.Cu) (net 2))
 (segment (start 154.1575 114.95) (end 153.728999 114.521499) (width 0.3) (layer F.Cu) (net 2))
 (segment (start 165.608 112.014) (end 168.91 112.014) (width 0.5) (layer F.Cu) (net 8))
 (via (at 168.91 112.014) (size 0.8) (drill 0.4) (layers F.Cu B.Cu) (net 8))
 (segment (start 167.132 111.252) (end 166.37 111.252) (width 0.5) (layer B.Cu) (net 8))
 (segment (start 166.37 111.252) (end 165.608 112.014) (width 0.5) (layer B.Cu) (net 8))
 (via (at 165.608 112.014) (size 0.8) (drill 0.4) (layers F.Cu B.Cu) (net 8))
 (segment (start 168.275 114.3) (end 168.275 112.395) (width 0.5) (layer F.Cu) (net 8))
 (segment (start 168.275 112.395) (end 167.132 111.252) (width 0.5) (layer F.Cu) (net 8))
 (via (at 167.132 111.252) (size 0.8) (drill 0.4) (layers F.Cu B.Cu) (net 8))
 (segment (start 140.716 126.746) (end 140.716 123.952) (width 0.5) (layer B.Cu) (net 8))
 (segment (start 140.716 123.952) (end 141.732 122.936) (width 0.5) (layer B.Cu) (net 8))
 (via (at 141.732 122.936) (size 0.8) (drill 0.4) (layers F.Cu B.Cu) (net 8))
 (segment (start 140.335 125.095) (end 140.335 126.365) (width 0.5) (layer F.Cu) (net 8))
 (segment (start 140.335 126.365) (end 140.716 126.746) (width 0.5) (layer F.Cu) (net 8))
 (via (at 140.716 126.746) (size 0.8) (drill 0.4) (layers F.Cu B.Cu) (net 8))
 (segment (start 157.48 112.268) (end 155.956 110.744) (width 0.5) (layer B.Cu) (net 8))
 (via (at 155.956 110.744) (size 0.8) (drill 0.4) (layers F.Cu B.Cu) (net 8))
 (segment (start 155.956 111.8235) (end 157.0355 111.8235) (width 0.5) (layer F.Cu) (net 8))
 (segment (start 157.0355 111.8235) (end 157.48 112.268) (width 0.5) (layer F.Cu) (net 8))
 (via (at 157.48 112.268) (size 0.8) (drill 0.4) (layers F.Cu B.Cu) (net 8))
 (segment (start 149.86 115.57) (end 148.844 115.57) (width 0.5) (layer F.Cu) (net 8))
 (segment (start 148.844 115.57) (end 148.59 115.316) (width 0.5) (layer F.Cu) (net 8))
 (via (at 148.59 115.316) (size 0.8) (drill 0.4) (layers F.Cu B.Cu) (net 8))
 (via (at 156.145 117.475) (size 0.8) (drill 0.4) (layers F.Cu B.Cu) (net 8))
 (via (at 156.145 116.625) (size 0.8) (drill 0.4) (layers F.Cu B.Cu) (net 8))
 (via (at 153.67 117.475) (size 0.8) (drill 0.4) (layers F.Cu B.Cu) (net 8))
 (via (at 154.495 117.475) (size 0.8) (drill 0.4) (layers F.Cu B.Cu) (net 8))
 (segment (start 156.145 116.625) (end 156.145 116.65) (width 0.3) (layer F.Cu) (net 8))
 (via (at 155.32 117.475) (size 0.8) (drill 0.4) (layers F.Cu B.Cu) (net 8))
 (via (at 155.32 116.625) (size 0.8) (drill 0.4) (layers F.Cu B.Cu) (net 8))
 (via (at 154.495 116.625) (size 0.8) (drill 0.4) (layers F.Cu B.Cu) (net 8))
 (via (at 153.67 116.625) (size 0.8) (drill 0.4) (layers F.Cu B.Cu) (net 8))
 (segment (start 139.7 121.61) (end 139.7 119.11) (width 0.3) (layer F.Cu) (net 8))
 (segment (start 142.4 119.41) (end 140 119.41) (width 0.3) (layer F.Cu) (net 8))
 (segment (start 140 119.41) (end 139.7 119.11) (width 0.3) (layer F.Cu) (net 8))
 (segment (start 139.7 117.11) (end 139.7 119.11) (width 0.3) (layer F.Cu) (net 8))
 (segment (start 157.157501 115.755501) (end 157.802499 115.755501) (width 1) (layer F.Cu) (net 1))
 (segment (start 157.802499 115.755501) (end 161.29 112.268) (width 1) (layer F.Cu) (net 1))
 (segment (start 161.29 112.268) (end 161.29 112.124) (width 1) (layer F.Cu) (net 1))
 (segment (start 157.157501 115.755501) (end 156.972 115.57) (width 0.8) (layer F.Cu) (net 1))
 (segment (start 156.972 115.57) (end 156.464 115.57) (width 0.8) (layer F.Cu) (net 1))
 (segment (start 157.157501 118.380001) (end 157.157501 115.755501) (width 0.8) (layer F.Cu) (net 1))
 (segment (start 156.21 115.57) (end 156.464 115.57) (width 0.3) (layer F.Cu) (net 1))
 (segment (start 156.18 115.6) (end 156.21 115.57) (width 0.3) (layer F.Cu) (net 1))
 (segment (start 156.1575 115.6) (end 156.18 115.6) (width 0.3) (layer F.Cu) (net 1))
 (segment (start 161.29 112.124) (end 161.18 112.124) (width 1) (layer F.Cu) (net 1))
 (segment (start 156.6 118.5) (end 157.037502 118.5) (width 0.8) (layer F.Cu) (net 1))
 (segment (start 157.037502 118.5) (end 157.157501 118.380001) (width 0.8) (layer F.Cu) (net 1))
 (segment (start 157.157501 118.380001) (end 157.037501 118.500001) (width 0.8) (layer F.Cu) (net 1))
 (segment (start 156.1575 118.5) (end 156.6 118.5) (width 0.3) (layer F.Cu) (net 1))
 (segment (start 155.6575 118.5) (end 155.6575 119.3355) (width 0.25) (layer F.Cu) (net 7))
 (segment (start 155.702 119.38) (end 155.702 119.3292) (width 0.25) (layer F.Cu) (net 7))
 (segment (start 155.6575 119.3355) (end 155.702 119.38) (width 0.3) (layer F.Cu) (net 7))
 (segment (start 159.385 123.0122) (end 155.702 119.3292) (width 0.4) (layer F.Cu) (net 7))
 (segment (start 159.385 123.19) (end 159.385 123.063) (width 0.4) (layer F.Cu) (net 7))
 (segment (start 159.3596 123.19) (end 159.385 123.19) (width 0.3) (layer F.Cu) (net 7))
 (segment (start 154.33548 123.19) (end 154.33548 123.28652) (width 0.5) (layer F.Cu) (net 6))
 (segment (start 154.33548 123.28652) (end 152.146 125.476) (width 0.5) (layer F.Cu) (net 6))
 (segment (start 152.146 125.476) (end 147.193 125.476) (width 0.5) (layer F.Cu) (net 6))
 (segment (start 155.16101 118.931745) (end 155.16101 119.902875) (width 0.25) (layer F.Cu) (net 6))
 (segment (start 155.16101 119.902875) (end 155.16101 119.22001) (width 0.25) (layer F.Cu) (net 6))
 (segment (start 154.33548 123.19) (end 154.33548 121.64032) (width 0.3) (layer F.Cu) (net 6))
 (segment (start 154.33548 121.64032) (end 155.16101 120.81479) (width 0.3) (layer F.Cu) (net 6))
 (segment (start 155.16101 120.81479) (end 155.16101 119.902875) (width 0.3) (layer F.Cu) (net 6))
 (segment (start 155.1575 118.5) (end 155.1575 118.928235) (width 0.25) (layer F.Cu) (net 6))
 (segment (start 155.1575 118.928235) (end 155.16101 118.931745) (width 0.25) (layer F.Cu) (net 6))
 (segment (start 154.33548 123.19) (end 154.36088 123.19) (width 1) (layer F.Cu) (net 6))
 (segment (start 154.36088 123.19) (end 156.39288 125.222) (width 1) (layer F.Cu) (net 6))
 (segment (start 156.39288 125.222) (end 161.544 125.222) (width 1) (layer F.Cu) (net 6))
 (segment (start 161.544 125.222) (end 162.546 124.22) (width 1) (layer F.Cu) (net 6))
 (segment (start 162.546 124.22) (end 162.546 122.95) (width 1) (layer F.Cu) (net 6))
 (segment (start 162.546 122.95) (end 163.696 121.8) (width 1) (layer F.Cu) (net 6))
 (segment (start 163.696 121.8) (end 168.275 121.8) (width 1) (layer F.Cu) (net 6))
 (segment (start 161.434 119.524) (end 163.71 121.8) (width 1) (layer F.Cu) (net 6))
 (segment (start 163.71 121.8) (end 168.275 121.8) (width 1) (layer F.Cu) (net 6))
 (segment (start 161.29 119.524) (end 161.434 119.524) (width 1) (layer F.Cu) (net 6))
 (segment (start 154.813 122.71248) (end 154.33548 123.19) (width 0.3) (layer F.Cu) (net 6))
 (segment (start 155.1575 122.36798) (end 154.33548 123.19) (width 0.3) (layer F.Cu) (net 6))
 (segment (start 146.685 119.38) (end 146.685 120.523) (width 0.5) (layer F.Cu) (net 9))
 (segment (start 146.685 120.523) (end 147.193 121.031) (width 0.5) (layer F.Cu) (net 9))
 (segment (start 147.193 121.031) (end 147.193 122.174) (width 0.5) (layer F.Cu) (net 9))
 (segment (start 154.6575 115.6) (end 154.6575 114.554018) (width 0.25) (layer F.Cu) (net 3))
 (segment (start 154.6575 114.554018) (end 154.657518 114.554) (width 0.25) (layer F.Cu) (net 3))
 (segment (start 154.657518 114.127018) (end 154.657518 114.554) (width 0.5) (layer F.Cu) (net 3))
 (segment (start 153.67 113.2205) (end 153.751 113.2205) (width 0.5) (layer F.Cu) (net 3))
 (segment (start 153.751 113.2205) (end 154.657518 114.127018) (width 0.5) (layer F.Cu) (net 3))
 (segment (start 153.6575 115.6) (end 151.795 115.6) (width 0.25) (layer F.Cu) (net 4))
 (segment (start 151.795 115.6) (end 151.765 115.57) (width 0.25) (layer F.Cu) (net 4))
 (segment (start 148.971 122.335) (end 150.08 123.444) (width 0.3) (layer F.Cu) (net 10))
 (segment (start 148.971 122.335) (end 148.971 119.507) (width 0.3) (layer F.Cu) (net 10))
 (segment (start 150.08 123.444) (end 151.13 123.444) (width 0.3) (layer F.Cu) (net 10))
 (segment (start 152.497 119.761) (end 154.209264 119.761) (width 0.3) (layer F.Cu) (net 5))
 (segment (start 154.209264 119.761) (end 154.653008 119.317256) (width 0.3) (layer F.Cu) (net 5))
 (segment (start 154.653008 119.317256) (end 154.653008 119.104492) (width 0.3) (layer F.Cu) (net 5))
 (segment (start 154.653008 119.104492) (end 154.6575 119.1) (width 0.3) (layer F.Cu) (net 5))
 (segment (start 151.13 119.444) (end 152.18 119.444) (width 0.3) (layer F.Cu) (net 5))
 (segment (start 152.18 119.444) (end 152.497 119.761) (width 0.3) (layer F.Cu) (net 5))
 (segment (start 154.6575 118.5) (end 154.6575 119.1) (width 0.25) (layer F.Cu) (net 5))
 (segment (start 151.32 119.634) (end 151.13 119.444) (width 0.3) (layer F.Cu) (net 5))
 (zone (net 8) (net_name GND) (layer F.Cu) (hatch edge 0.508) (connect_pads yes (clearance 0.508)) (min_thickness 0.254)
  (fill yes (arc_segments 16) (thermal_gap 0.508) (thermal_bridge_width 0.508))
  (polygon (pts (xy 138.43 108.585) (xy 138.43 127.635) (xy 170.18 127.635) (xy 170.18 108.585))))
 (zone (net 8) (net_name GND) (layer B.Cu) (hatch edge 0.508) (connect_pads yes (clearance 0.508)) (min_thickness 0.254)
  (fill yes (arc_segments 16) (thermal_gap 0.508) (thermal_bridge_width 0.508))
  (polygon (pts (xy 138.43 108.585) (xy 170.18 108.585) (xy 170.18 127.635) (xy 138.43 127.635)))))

